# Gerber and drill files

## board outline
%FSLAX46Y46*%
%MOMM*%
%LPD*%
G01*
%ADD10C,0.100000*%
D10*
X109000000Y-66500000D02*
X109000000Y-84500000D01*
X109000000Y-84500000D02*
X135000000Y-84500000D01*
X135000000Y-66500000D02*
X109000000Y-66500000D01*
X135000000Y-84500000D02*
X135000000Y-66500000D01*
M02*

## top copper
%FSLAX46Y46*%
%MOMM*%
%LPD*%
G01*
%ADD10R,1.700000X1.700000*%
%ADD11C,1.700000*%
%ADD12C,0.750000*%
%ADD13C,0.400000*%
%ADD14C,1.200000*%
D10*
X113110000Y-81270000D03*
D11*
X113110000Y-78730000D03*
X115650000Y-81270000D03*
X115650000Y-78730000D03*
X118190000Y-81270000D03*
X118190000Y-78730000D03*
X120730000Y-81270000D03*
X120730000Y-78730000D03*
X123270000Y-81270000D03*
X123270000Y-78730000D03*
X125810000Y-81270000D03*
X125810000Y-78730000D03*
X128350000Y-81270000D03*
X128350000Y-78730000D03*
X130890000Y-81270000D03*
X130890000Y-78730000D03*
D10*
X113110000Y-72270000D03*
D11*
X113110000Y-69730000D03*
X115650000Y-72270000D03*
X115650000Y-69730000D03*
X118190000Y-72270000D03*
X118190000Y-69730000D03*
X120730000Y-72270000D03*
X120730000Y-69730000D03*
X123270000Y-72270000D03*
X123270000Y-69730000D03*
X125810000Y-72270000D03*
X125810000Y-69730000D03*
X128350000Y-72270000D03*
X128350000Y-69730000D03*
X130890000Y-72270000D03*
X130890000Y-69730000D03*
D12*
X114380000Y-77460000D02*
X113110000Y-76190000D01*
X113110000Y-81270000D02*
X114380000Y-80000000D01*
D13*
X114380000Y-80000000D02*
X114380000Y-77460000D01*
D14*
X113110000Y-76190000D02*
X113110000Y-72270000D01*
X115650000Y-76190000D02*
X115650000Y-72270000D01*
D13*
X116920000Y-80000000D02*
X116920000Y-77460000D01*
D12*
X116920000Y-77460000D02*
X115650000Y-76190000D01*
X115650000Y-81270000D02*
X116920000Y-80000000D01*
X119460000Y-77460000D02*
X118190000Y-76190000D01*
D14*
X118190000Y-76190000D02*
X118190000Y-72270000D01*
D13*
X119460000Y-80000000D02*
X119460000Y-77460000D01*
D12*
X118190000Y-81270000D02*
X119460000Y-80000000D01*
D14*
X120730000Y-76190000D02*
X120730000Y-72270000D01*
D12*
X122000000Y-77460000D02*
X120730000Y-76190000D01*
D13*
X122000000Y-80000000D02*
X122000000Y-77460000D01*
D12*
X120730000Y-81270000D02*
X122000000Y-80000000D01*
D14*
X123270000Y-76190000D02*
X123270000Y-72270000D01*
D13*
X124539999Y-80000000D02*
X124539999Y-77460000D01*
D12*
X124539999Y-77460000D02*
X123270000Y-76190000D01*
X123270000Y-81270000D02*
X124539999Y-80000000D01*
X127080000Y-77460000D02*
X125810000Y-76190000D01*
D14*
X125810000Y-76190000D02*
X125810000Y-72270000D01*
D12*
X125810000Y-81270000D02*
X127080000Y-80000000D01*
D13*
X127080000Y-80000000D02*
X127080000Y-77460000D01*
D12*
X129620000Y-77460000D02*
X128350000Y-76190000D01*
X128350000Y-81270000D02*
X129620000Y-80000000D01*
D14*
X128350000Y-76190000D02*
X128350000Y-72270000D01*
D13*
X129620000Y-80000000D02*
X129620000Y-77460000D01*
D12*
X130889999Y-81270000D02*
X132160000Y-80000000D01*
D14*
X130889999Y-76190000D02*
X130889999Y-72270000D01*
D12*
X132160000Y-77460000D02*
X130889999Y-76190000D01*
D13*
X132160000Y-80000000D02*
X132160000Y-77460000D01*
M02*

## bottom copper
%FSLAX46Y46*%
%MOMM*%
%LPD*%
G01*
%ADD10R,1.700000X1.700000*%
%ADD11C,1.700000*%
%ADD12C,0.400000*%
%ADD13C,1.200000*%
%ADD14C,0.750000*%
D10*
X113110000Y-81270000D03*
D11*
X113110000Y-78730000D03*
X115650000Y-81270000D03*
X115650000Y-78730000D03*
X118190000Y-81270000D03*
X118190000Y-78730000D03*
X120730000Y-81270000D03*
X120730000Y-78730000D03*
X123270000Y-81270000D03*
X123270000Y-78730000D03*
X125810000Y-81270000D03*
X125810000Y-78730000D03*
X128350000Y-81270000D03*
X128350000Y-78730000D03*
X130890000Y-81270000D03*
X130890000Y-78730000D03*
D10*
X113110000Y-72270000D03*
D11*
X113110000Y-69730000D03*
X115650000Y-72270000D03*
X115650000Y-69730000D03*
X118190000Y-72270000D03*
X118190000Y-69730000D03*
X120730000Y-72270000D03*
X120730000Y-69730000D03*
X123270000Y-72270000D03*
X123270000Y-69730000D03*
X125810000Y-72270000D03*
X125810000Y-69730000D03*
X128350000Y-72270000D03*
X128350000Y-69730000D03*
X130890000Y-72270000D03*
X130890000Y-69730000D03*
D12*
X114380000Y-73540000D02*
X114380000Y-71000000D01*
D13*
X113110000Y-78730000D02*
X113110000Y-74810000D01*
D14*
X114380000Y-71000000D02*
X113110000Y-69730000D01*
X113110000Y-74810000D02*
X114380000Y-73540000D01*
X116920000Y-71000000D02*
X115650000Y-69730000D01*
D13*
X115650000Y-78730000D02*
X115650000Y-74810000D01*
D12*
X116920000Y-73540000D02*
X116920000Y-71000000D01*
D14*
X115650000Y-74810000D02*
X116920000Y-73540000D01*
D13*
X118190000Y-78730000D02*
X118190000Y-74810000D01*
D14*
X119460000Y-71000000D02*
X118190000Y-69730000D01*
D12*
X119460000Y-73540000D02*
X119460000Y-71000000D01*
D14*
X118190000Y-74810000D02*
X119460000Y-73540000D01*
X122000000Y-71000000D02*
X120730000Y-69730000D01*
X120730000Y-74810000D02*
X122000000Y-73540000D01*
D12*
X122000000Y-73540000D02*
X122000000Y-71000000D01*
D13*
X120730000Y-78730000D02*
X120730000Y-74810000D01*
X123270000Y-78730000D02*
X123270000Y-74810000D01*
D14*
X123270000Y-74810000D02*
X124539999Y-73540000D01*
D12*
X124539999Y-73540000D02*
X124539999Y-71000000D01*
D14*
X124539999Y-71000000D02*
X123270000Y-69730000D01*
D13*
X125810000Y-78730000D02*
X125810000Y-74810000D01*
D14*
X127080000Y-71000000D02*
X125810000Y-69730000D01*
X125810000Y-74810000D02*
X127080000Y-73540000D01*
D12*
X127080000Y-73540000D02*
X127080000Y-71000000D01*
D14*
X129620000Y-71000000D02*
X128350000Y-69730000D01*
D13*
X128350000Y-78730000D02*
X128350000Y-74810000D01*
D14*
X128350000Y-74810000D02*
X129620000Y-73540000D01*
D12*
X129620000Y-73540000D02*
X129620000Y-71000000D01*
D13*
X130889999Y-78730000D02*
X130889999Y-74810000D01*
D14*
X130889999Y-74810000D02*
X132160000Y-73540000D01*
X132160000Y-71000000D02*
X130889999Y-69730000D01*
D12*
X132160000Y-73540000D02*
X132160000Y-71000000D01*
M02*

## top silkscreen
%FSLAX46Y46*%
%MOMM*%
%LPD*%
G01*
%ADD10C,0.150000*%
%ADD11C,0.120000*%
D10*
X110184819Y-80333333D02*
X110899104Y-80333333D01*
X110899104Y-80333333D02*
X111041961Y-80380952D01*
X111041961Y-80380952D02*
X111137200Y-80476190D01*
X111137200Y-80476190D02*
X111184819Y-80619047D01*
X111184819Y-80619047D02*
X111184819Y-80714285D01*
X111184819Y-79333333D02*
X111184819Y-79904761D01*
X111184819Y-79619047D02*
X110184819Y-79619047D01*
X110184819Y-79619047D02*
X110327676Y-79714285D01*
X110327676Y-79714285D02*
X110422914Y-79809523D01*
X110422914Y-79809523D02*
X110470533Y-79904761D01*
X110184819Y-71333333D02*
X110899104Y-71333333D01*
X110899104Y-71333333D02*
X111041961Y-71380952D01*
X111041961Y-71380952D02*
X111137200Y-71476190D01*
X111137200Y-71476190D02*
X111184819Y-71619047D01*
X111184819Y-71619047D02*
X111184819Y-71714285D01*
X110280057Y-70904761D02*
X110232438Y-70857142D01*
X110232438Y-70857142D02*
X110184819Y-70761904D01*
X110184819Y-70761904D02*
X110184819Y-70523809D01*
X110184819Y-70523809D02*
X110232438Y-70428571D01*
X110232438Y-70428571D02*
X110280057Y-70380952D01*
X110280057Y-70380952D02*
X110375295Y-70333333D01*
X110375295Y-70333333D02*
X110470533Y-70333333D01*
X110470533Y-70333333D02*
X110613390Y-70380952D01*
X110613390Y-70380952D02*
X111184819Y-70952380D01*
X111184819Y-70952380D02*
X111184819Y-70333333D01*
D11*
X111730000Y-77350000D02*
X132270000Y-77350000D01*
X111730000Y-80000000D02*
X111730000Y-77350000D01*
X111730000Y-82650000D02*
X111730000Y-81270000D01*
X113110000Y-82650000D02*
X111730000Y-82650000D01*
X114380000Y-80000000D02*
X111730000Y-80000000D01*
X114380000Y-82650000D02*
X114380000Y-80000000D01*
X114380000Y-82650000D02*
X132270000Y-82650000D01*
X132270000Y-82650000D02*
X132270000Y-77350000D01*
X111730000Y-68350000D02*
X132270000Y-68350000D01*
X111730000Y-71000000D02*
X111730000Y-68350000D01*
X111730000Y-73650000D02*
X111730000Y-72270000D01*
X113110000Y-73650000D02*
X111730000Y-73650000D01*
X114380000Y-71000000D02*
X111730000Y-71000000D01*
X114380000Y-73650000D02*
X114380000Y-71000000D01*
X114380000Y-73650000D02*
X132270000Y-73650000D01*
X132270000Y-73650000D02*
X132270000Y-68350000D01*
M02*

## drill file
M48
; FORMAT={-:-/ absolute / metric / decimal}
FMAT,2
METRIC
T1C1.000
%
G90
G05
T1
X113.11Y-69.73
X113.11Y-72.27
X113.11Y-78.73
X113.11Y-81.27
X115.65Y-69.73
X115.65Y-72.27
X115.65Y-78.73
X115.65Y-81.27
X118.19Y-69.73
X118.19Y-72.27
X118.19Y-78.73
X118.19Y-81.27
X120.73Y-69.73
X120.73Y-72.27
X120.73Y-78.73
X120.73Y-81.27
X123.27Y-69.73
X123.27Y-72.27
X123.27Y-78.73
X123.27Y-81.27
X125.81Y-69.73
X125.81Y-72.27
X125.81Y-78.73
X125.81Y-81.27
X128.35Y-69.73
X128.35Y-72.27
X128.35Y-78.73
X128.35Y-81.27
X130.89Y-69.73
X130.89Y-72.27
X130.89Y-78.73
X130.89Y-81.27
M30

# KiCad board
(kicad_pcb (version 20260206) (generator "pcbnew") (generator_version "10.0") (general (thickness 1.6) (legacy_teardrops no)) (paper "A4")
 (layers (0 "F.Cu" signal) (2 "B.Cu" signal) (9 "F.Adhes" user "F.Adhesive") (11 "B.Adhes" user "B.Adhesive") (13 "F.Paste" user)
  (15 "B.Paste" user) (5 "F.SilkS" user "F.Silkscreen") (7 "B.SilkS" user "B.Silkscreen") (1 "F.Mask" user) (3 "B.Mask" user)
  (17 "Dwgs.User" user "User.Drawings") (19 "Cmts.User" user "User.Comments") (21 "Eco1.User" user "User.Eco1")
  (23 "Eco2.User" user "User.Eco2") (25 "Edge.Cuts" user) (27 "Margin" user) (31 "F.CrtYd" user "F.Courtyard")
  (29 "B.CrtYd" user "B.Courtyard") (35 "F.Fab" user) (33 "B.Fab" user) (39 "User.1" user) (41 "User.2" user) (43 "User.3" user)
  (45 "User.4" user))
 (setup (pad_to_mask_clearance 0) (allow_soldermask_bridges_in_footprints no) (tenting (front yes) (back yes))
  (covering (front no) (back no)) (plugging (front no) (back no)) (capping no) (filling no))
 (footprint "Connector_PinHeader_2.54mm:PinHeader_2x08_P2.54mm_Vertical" (layer "F.Cu") (at 113.11 81.27 90)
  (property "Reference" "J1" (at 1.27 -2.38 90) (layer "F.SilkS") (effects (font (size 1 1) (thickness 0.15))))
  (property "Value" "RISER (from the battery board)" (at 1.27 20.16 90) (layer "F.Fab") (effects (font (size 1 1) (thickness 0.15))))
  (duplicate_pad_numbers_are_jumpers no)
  (fp_line (start 3.92 -1.38) (end 3.92 19.16) (stroke (width 0.12) (type solid)) (layer "F.SilkS"))
  (fp_line (start 1.27 -1.38) (end 3.92 -1.38) (stroke (width 0.12) (type solid)) (layer "F.SilkS"))
  (fp_line (start -1.38 -1.38) (end 0 -1.38) (stroke (width 0.12) (type solid)) (layer "F.SilkS"))
  (fp_line (start -1.38 0) (end -1.38 -1.38) (stroke (width 0.12) (type solid)) (layer "F.SilkS"))
  (fp_line (start 1.27 1.27) (end 1.27 -1.38) (stroke (width 0.12) (type solid)) (layer "F.SilkS"))
  (fp_line (start -1.38 1.27) (end 1.27 1.27) (stroke (width 0.12) (type solid)) (layer "F.SilkS"))
  (fp_line (start -1.38 1.27) (end -1.38 19.16) (stroke (width 0.12) (type solid)) (layer "F.SilkS"))
  (fp_line (start -1.38 19.16) (end 3.92 19.16) (stroke (width 0.12) (type solid)) (layer "F.SilkS"))
  (pad "1" thru_hole rect (at 0 0 90) (size 1.7 1.7) (drill 1) (layers "*.Cu" "*.Mask") (remove_unused_layers no) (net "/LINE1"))
  (pad "2" thru_hole circle (at 2.54 0 90) (size 1.7 1.7) (drill 1) (layers "*.Cu" "*.Mask") (remove_unused_layers no) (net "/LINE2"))
  (pad "3" thru_hole circle (at 0 2.54 90) (size 1.7 1.7) (drill 1) (layers "*.Cu" "*.Mask") (remove_unused_layers no) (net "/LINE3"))
  (pad "4" thru_hole circle (at 2.54 2.54 90) (size 1.7 1.7) (drill 1) (layers "*.Cu" "*.Mask") (remove_unused_layers no) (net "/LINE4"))
  (pad "5" thru_hole circle (at 0 5.08 90) (size 1.7 1.7) (drill 1) (layers "*.Cu" "*.Mask") (remove_unused_layers no) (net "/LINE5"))
  (pad "6" thru_hole circle (at 2.54 5.08 90) (size 1.7 1.7) (drill 1) (layers "*.Cu" "*.Mask") (remove_unused_layers no) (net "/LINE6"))
  (pad "7" thru_hole circle (at 0 7.62 90) (size 1.7 1.7) (drill 1) (layers "*.Cu" "*.Mask") (remove_unused_layers no) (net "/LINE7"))
  (pad "8" thru_hole circle (at 2.54 7.62 90) (size 1.7 1.7) (drill 1) (layers "*.Cu" "*.Mask") (remove_unused_layers no) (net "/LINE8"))
  (pad "9" thru_hole circle (at 0 10.16 90) (size 1.7 1.7) (drill 1) (layers "*.Cu" "*.Mask") (remove_unused_layers no) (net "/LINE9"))
  (pad "10" thru_hole circle (at 2.54 10.16 90) (size 1.7 1.7) (drill 1) (layers "*.Cu" "*.Mask") (remove_unused_layers no) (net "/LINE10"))
  (pad "11" thru_hole circle (at 0 12.7 90) (size 1.7 1.7) (drill 1) (layers "*.Cu" "*.Mask") (remove_unused_layers no) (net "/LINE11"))
  (pad "12" thru_hole circle (at 2.54 12.7 90) (size 1.7 1.7) (drill 1) (layers "*.Cu" "*.Mask") (remove_unused_layers no) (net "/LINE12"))
  (pad "13" thru_hole circle (at 0 15.24 90) (size 1.7 1.7) (drill 1) (layers "*.Cu" "*.Mask") (remove_unused_layers no) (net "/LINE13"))
  (pad "14" thru_hole circle (at 2.54 15.24 90) (size 1.7 1.7) (drill 1) (layers "*.Cu" "*.Mask") (remove_unused_layers no) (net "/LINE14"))
  (pad "15" thru_hole circle (at 0 17.78 90) (size 1.7 1.7) (drill 1) (layers "*.Cu" "*.Mask") (remove_unused_layers no) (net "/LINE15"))
  (pad "16" thru_hole circle (at 2.54 17.78 90) (size 1.7 1.7) (drill 1) (layers "*.Cu" "*.Mask") (remove_unused_layers no) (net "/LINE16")))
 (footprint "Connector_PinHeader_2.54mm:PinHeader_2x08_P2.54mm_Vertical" (layer "F.Cu") (at 113.11 72.27 90)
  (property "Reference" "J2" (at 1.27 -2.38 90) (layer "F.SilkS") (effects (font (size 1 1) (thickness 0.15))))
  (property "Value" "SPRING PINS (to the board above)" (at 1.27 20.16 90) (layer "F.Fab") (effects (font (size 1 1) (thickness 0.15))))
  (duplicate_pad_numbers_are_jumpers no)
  (fp_line (start 3.92 -1.38) (end 3.92 19.16) (stroke (width 0.12) (type solid)) (layer "F.SilkS"))
  (fp_line (start 1.27 -1.38) (end 3.92 -1.38) (stroke (width 0.12) (type solid)) (layer "F.SilkS"))
  (fp_line (start -1.38 -1.38) (end 0 -1.38) (stroke (width 0.12) (type solid)) (layer "F.SilkS"))
  (fp_line (start -1.38 0) (end -1.38 -1.38) (stroke (width 0.12) (type solid)) (layer "F.SilkS"))
  (fp_line (start 1.27 1.27) (end 1.27 -1.38) (stroke (width 0.12) (type solid)) (layer "F.SilkS"))
  (fp_line (start -1.38 1.27) (end 1.27 1.27) (stroke (width 0.12) (type solid)) (layer "F.SilkS"))
  (fp_line (start -1.38 1.27) (end -1.38 19.16) (stroke (width 0.12) (type solid)) (layer "F.SilkS"))
  (fp_line (start -1.38 19.16) (end 3.92 19.16) (stroke (width 0.12) (type solid)) (layer "F.SilkS"))
  (pad "1" thru_hole rect (at 0 0 90) (size 1.7 1.7) (drill 1) (layers "*.Cu" "*.Mask") (remove_unused_layers no) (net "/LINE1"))
  (pad "2" thru_hole circle (at 2.54 0 90) (size 1.7 1.7) (drill 1) (layers "*.Cu" "*.Mask") (remove_unused_layers no) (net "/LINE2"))
  (pad "3" thru_hole circle (at 0 2.54 90) (size 1.7 1.7) (drill 1) (layers "*.Cu" "*.Mask") (remove_unused_layers no) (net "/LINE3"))
  (pad "4" thru_hole circle (at 2.54 2.54 90) (size 1.7 1.7) (drill 1) (layers "*.Cu" "*.Mask") (remove_unused_layers no) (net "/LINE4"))
  (pad "5" thru_hole circle (at 0 5.08 90) (size 1.7 1.7) (drill 1) (layers "*.Cu" "*.Mask") (remove_unused_layers no) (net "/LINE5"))
  (pad "6" thru_hole circle (at 2.54 5.08 90) (size 1.7 1.7) (drill 1) (layers "*.Cu" "*.Mask") (remove_unused_layers no) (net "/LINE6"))
  (pad "7" thru_hole circle (at 0 7.62 90) (size 1.7 1.7) (drill 1) (layers "*.Cu" "*.Mask") (remove_unused_layers no) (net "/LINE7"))
  (pad "8" thru_hole circle (at 2.54 7.62 90) (size 1.7 1.7) (drill 1) (layers "*.Cu" "*.Mask") (remove_unused_layers no) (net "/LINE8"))
  (pad "9" thru_hole circle (at 0 10.16 90) (size 1.7 1.7) (drill 1) (layers "*.Cu" "*.Mask") (remove_unused_layers no) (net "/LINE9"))
  (pad "10" thru_hole circle (at 2.54 10.16 90) (size 1.7 1.7) (drill 1) (layers "*.Cu" "*.Mask") (remove_unused_layers no) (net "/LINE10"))
  (pad "11" thru_hole circle (at 0 12.7 90) (size 1.7 1.7) (drill 1) (layers "*.Cu" "*.Mask") (remove_unused_layers no) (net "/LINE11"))
  (pad "12" thru_hole circle (at 2.54 12.7 90) (size 1.7 1.7) (drill 1) (layers "*.Cu" "*.Mask") (remove_unused_layers no) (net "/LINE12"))
  (pad "13" thru_hole circle (at 0 15.24 90) (size 1.7 1.7) (drill 1) (layers "*.Cu" "*.Mask") (remove_unused_layers no) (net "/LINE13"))
  (pad "14" thru_hole circle (at 2.54 15.24 90) (size 1.7 1.7) (drill 1) (layers "*.Cu" "*.Mask") (remove_unused_layers no) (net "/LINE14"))
  (pad "15" thru_hole circle (at 0 17.78 90) (size 1.7 1.7) (drill 1) (layers "*.Cu" "*.Mask") (remove_unused_layers no) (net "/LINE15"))
  (pad "16" thru_hole circle (at 2.54 17.78 90) (size 1.7 1.7) (drill 1) (layers "*.Cu" "*.Mask") (remove_unused_layers no) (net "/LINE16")))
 (gr_line (start 109 66.5) (end 109 84.5) (stroke (width 0.1) (type default)) (layer "Edge.Cuts"))
 (gr_line (start 109 84.5) (end 135 84.5) (stroke (width 0.1) (type default)) (layer "Edge.Cuts"))
 (gr_line (start 135 66.5) (end 109 66.5) (stroke (width 0.1) (type default)) (layer "Edge.Cuts"))
 (gr_line (start 135 84.5) (end 135 66.5) (stroke (width 0.1) (type default)) (layer "Edge.Cuts"))
 (segment (start 114.38 77.46) (end 113.11 76.19) (width 0.75) (locked yes) (layer "F.Cu") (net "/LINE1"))
 (segment (start 113.11 81.27) (end 114.38 80) (width 0.75) (locked yes) (layer "F.Cu") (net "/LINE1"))
 (segment (start 114.38 80) (end 114.38 77.46) (width 0.4) (locked yes) (layer "F.Cu") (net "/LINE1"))
 (segment (start 113.11 76.19) (end 113.11 72.27) (width 1.2) (locked yes) (layer "F.Cu") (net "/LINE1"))
 (segment (start 114.38 73.54) (end 114.38 71) (width 0.4) (locked yes) (layer "B.Cu") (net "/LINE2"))
 (segment (start 113.11 78.73) (end 113.11 74.81) (width 1.2) (locked yes) (layer "B.Cu") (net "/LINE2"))
 (segment (start 114.38 71) (end 113.11 69.73) (width 0.75) (locked yes) (layer "B.Cu") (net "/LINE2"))
 (segment (start 113.11 74.81) (end 114.38 73.54) (width 0.75) (locked yes) (layer "B.Cu") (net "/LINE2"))
 (segment (start 115.65 76.19) (end 115.65 72.27) (width 1.2) (locked yes) (layer "F.Cu") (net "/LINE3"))
 (segment (start 116.92 80) (end 116.92 77.46) (width 0.4) (locked yes) (layer "F.Cu") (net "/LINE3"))
 (segment (start 116.92 77.46) (end 115.65 76.19) (width 0.75) (locked yes) (layer "F.Cu") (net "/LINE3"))
 (segment (start 115.65 81.27) (end 116.92 80) (width 0.75) (locked yes) (layer "F.Cu") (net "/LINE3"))
 (segment (start 116.92 71) (end 115.65 69.73) (width 0.75) (locked yes) (layer "B.Cu") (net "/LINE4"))
 (segment (start 115.65 78.73) (end 115.65 74.81) (width 1.2) (locked yes) (layer "B.Cu") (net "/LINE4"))
 (segment (start 116.92 73.54) (end 116.92 71) (width 0.4) (locked yes) (layer "B.Cu") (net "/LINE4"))
 (segment (start 115.65 74.81) (end 116.92 73.54) (width 0.75) (locked yes) (layer "B.Cu") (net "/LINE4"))
 (segment (start 119.46 77.46) (end 118.19 76.19) (width 0.75) (locked yes) (layer "F.Cu") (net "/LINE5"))
 (segment (start 118.19 76.19) (end 118.19 72.27) (width 1.2) (locked yes) (layer "F.Cu") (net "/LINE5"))
 (segment (start 119.46 80) (end 119.46 77.46) (width 0.4) (locked yes) (layer "F.Cu") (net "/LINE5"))
 (segment (start 118.19 81.27) (end 119.46 80) (width 0.75) (locked yes) (layer "F.Cu") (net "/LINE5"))
 (segment (start 118.19 78.73) (end 118.19 74.81) (width 1.2) (locked yes) (layer "B.Cu") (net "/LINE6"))
 (segment (start 119.46 71) (end 118.19 69.73) (width 0.75) (locked yes) (layer "B.Cu") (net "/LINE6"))
 (segment (start 119.46 73.54) (end 119.46 71) (width 0.4) (locked yes) (layer "B.Cu") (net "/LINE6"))
 (segment (start 118.19 74.81) (end 119.46 73.54) (width 0.75) (locked yes) (layer "B.Cu") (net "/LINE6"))
 (segment (start 120.73 76.19) (end 120.73 72.27) (width 1.2) (locked yes) (layer "F.Cu") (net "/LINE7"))
 (segment (start 122 77.46) (end 120.73 76.19) (width 0.75) (locked yes) (layer "F.Cu") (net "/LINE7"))
 (segment (start 122 80) (end 122 77.46) (width 0.4) (locked yes) (layer "F.Cu") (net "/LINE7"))
 (segment (start 120.73 81.27) (end 122 80) (width 0.75) (locked yes) (layer "F.Cu") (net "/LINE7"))
 (segment (start 122 71) (end 120.73 69.73) (width 0.75) (locked yes) (layer "B.Cu") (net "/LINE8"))
 (segment (start 120.73 74.81) (end 122 73.54) (width 0.75) (locked yes) (layer "B.Cu") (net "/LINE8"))
 (segment (start 122 73.54) (end 122 71) (width 0.4) (locked yes) (layer "B.Cu") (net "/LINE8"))
 (segment (start 120.73 78.73) (end 120.73 74.81) (width 1.2) (locked yes) (layer "B.Cu") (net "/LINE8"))
 (segment (start 123.27 76.19) (end 123.27 72.27) (width 1.2) (locked yes) (layer "F.Cu") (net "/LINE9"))
 (segment (start 124.539999 80) (end 124.539999 77.46) (width 0.4) (locked yes) (layer "F.Cu") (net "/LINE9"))
 (segment (start 124.539999 77.46) (end 123.27 76.19) (width 0.75) (locked yes) (layer "F.Cu") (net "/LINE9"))
 (segment (start 123.27 81.27) (end 124.539999 80) (width 0.75) (locked yes) (layer "F.Cu") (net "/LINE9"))
 (segment (start 123.27 78.73) (end 123.27 74.81) (width 1.2) (locked yes) (layer "B.Cu") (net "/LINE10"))
 (segment (start 123.27 74.81) (end 124.539999 73.54) (width 0.75) (locked yes) (layer "B.Cu") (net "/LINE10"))
 (segment (start 124.539999 73.54) (end 124.539999 71) (width 0.4) (locked yes) (layer "B.Cu") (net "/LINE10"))
 (segment (start 124.539999 71) (end 123.27 69.73) (width 0.75) (locked yes) (layer "B.Cu") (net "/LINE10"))
 (segment (start 127.08 77.46) (end 125.81 76.19) (width 0.75) (locked yes) (layer "F.Cu") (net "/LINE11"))
 (segment (start 125.81 76.19) (end 125.81 72.27) (width 1.2) (locked yes) (layer "F.Cu") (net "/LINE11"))
 (segment (start 125.81 81.27) (end 127.08 80) (width 0.75) (locked yes) (layer "F.Cu") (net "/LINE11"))
 (segment (start 127.08 80) (end 127.08 77.46) (width 0.4) (locked yes) (layer "F.Cu") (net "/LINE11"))
 (segment (start 125.81 78.73) (end 125.81 74.81) (width 1.2) (locked yes) (layer "B.Cu") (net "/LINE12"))
 (segment (start 127.08 71) (end 125.81 69.73) (width 0.75) (locked yes) (layer "B.Cu") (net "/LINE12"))
 (segment (start 125.81 74.81) (end 127.08 73.54) (width 0.75) (locked yes) (layer "B.Cu") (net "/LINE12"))
 (segment (start 127.08 73.54) (end 127.08 71) (width 0.4) (locked yes) (layer "B.Cu") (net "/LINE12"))
 (segment (start 129.62 77.46) (end 128.35 76.19) (width 0.75) (locked yes) (layer "F.Cu") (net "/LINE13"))
 (segment (start 128.35 81.27) (end 129.62 80) (width 0.75) (locked yes) (layer "F.Cu") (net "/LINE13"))
 (segment (start 128.35 76.19) (end 128.35 72.27) (width 1.2) (locked yes) (layer "F.Cu") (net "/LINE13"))
 (segment (start 129.62 80) (end 129.62 77.46) (width 0.4) (locked yes) (layer "F.Cu") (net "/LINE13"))
 (segment (start 129.62 71) (end 128.35 69.73) (width 0.75) (locked yes) (layer "B.Cu") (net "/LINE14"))
 (segment (start 128.35 78.73) (end 128.35 74.81) (width 1.2) (locked yes) (layer "B.Cu") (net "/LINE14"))
 (segment (start 128.35 74.81) (end 129.62 73.54) (width 0.75) (locked yes) (layer "B.Cu") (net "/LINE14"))
 (segment (start 129.62 73.54) (end 129.62 71) (width 0.4) (locked yes) (layer "B.Cu") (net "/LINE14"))
 (segment (start 130.889999 81.27) (end 132.16 80) (width 0.75) (locked yes) (layer "F.Cu") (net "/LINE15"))
 (segment (start 130.889999 76.19) (end 130.889999 72.27) (width 1.2) (locked yes) (layer "F.Cu") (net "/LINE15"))
 (segment (start 132.16 77.46) (end 130.889999 76.19) (width 0.75) (locked yes) (layer "F.Cu") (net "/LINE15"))
 (segment (start 132.16 80) (end 132.16 77.46) (width 0.4) (locked yes) (layer "F.Cu") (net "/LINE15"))
 (segment (start 130.889999 78.73) (end 130.889999 74.81) (width 1.2) (locked yes) (layer "B.Cu") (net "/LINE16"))
 (segment (start 130.889999 74.81) (end 132.16 73.54) (width 0.75) (locked yes) (layer "B.Cu") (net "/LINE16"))
 (segment (start 132.16 71) (end 130.889999 69.73) (width 0.75) (locked yes) (layer "B.Cu") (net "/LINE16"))
 (segment (start 132.16 73.54) (end 132.16 71) (width 0.4) (locked yes) (layer "B.Cu") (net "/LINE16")))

